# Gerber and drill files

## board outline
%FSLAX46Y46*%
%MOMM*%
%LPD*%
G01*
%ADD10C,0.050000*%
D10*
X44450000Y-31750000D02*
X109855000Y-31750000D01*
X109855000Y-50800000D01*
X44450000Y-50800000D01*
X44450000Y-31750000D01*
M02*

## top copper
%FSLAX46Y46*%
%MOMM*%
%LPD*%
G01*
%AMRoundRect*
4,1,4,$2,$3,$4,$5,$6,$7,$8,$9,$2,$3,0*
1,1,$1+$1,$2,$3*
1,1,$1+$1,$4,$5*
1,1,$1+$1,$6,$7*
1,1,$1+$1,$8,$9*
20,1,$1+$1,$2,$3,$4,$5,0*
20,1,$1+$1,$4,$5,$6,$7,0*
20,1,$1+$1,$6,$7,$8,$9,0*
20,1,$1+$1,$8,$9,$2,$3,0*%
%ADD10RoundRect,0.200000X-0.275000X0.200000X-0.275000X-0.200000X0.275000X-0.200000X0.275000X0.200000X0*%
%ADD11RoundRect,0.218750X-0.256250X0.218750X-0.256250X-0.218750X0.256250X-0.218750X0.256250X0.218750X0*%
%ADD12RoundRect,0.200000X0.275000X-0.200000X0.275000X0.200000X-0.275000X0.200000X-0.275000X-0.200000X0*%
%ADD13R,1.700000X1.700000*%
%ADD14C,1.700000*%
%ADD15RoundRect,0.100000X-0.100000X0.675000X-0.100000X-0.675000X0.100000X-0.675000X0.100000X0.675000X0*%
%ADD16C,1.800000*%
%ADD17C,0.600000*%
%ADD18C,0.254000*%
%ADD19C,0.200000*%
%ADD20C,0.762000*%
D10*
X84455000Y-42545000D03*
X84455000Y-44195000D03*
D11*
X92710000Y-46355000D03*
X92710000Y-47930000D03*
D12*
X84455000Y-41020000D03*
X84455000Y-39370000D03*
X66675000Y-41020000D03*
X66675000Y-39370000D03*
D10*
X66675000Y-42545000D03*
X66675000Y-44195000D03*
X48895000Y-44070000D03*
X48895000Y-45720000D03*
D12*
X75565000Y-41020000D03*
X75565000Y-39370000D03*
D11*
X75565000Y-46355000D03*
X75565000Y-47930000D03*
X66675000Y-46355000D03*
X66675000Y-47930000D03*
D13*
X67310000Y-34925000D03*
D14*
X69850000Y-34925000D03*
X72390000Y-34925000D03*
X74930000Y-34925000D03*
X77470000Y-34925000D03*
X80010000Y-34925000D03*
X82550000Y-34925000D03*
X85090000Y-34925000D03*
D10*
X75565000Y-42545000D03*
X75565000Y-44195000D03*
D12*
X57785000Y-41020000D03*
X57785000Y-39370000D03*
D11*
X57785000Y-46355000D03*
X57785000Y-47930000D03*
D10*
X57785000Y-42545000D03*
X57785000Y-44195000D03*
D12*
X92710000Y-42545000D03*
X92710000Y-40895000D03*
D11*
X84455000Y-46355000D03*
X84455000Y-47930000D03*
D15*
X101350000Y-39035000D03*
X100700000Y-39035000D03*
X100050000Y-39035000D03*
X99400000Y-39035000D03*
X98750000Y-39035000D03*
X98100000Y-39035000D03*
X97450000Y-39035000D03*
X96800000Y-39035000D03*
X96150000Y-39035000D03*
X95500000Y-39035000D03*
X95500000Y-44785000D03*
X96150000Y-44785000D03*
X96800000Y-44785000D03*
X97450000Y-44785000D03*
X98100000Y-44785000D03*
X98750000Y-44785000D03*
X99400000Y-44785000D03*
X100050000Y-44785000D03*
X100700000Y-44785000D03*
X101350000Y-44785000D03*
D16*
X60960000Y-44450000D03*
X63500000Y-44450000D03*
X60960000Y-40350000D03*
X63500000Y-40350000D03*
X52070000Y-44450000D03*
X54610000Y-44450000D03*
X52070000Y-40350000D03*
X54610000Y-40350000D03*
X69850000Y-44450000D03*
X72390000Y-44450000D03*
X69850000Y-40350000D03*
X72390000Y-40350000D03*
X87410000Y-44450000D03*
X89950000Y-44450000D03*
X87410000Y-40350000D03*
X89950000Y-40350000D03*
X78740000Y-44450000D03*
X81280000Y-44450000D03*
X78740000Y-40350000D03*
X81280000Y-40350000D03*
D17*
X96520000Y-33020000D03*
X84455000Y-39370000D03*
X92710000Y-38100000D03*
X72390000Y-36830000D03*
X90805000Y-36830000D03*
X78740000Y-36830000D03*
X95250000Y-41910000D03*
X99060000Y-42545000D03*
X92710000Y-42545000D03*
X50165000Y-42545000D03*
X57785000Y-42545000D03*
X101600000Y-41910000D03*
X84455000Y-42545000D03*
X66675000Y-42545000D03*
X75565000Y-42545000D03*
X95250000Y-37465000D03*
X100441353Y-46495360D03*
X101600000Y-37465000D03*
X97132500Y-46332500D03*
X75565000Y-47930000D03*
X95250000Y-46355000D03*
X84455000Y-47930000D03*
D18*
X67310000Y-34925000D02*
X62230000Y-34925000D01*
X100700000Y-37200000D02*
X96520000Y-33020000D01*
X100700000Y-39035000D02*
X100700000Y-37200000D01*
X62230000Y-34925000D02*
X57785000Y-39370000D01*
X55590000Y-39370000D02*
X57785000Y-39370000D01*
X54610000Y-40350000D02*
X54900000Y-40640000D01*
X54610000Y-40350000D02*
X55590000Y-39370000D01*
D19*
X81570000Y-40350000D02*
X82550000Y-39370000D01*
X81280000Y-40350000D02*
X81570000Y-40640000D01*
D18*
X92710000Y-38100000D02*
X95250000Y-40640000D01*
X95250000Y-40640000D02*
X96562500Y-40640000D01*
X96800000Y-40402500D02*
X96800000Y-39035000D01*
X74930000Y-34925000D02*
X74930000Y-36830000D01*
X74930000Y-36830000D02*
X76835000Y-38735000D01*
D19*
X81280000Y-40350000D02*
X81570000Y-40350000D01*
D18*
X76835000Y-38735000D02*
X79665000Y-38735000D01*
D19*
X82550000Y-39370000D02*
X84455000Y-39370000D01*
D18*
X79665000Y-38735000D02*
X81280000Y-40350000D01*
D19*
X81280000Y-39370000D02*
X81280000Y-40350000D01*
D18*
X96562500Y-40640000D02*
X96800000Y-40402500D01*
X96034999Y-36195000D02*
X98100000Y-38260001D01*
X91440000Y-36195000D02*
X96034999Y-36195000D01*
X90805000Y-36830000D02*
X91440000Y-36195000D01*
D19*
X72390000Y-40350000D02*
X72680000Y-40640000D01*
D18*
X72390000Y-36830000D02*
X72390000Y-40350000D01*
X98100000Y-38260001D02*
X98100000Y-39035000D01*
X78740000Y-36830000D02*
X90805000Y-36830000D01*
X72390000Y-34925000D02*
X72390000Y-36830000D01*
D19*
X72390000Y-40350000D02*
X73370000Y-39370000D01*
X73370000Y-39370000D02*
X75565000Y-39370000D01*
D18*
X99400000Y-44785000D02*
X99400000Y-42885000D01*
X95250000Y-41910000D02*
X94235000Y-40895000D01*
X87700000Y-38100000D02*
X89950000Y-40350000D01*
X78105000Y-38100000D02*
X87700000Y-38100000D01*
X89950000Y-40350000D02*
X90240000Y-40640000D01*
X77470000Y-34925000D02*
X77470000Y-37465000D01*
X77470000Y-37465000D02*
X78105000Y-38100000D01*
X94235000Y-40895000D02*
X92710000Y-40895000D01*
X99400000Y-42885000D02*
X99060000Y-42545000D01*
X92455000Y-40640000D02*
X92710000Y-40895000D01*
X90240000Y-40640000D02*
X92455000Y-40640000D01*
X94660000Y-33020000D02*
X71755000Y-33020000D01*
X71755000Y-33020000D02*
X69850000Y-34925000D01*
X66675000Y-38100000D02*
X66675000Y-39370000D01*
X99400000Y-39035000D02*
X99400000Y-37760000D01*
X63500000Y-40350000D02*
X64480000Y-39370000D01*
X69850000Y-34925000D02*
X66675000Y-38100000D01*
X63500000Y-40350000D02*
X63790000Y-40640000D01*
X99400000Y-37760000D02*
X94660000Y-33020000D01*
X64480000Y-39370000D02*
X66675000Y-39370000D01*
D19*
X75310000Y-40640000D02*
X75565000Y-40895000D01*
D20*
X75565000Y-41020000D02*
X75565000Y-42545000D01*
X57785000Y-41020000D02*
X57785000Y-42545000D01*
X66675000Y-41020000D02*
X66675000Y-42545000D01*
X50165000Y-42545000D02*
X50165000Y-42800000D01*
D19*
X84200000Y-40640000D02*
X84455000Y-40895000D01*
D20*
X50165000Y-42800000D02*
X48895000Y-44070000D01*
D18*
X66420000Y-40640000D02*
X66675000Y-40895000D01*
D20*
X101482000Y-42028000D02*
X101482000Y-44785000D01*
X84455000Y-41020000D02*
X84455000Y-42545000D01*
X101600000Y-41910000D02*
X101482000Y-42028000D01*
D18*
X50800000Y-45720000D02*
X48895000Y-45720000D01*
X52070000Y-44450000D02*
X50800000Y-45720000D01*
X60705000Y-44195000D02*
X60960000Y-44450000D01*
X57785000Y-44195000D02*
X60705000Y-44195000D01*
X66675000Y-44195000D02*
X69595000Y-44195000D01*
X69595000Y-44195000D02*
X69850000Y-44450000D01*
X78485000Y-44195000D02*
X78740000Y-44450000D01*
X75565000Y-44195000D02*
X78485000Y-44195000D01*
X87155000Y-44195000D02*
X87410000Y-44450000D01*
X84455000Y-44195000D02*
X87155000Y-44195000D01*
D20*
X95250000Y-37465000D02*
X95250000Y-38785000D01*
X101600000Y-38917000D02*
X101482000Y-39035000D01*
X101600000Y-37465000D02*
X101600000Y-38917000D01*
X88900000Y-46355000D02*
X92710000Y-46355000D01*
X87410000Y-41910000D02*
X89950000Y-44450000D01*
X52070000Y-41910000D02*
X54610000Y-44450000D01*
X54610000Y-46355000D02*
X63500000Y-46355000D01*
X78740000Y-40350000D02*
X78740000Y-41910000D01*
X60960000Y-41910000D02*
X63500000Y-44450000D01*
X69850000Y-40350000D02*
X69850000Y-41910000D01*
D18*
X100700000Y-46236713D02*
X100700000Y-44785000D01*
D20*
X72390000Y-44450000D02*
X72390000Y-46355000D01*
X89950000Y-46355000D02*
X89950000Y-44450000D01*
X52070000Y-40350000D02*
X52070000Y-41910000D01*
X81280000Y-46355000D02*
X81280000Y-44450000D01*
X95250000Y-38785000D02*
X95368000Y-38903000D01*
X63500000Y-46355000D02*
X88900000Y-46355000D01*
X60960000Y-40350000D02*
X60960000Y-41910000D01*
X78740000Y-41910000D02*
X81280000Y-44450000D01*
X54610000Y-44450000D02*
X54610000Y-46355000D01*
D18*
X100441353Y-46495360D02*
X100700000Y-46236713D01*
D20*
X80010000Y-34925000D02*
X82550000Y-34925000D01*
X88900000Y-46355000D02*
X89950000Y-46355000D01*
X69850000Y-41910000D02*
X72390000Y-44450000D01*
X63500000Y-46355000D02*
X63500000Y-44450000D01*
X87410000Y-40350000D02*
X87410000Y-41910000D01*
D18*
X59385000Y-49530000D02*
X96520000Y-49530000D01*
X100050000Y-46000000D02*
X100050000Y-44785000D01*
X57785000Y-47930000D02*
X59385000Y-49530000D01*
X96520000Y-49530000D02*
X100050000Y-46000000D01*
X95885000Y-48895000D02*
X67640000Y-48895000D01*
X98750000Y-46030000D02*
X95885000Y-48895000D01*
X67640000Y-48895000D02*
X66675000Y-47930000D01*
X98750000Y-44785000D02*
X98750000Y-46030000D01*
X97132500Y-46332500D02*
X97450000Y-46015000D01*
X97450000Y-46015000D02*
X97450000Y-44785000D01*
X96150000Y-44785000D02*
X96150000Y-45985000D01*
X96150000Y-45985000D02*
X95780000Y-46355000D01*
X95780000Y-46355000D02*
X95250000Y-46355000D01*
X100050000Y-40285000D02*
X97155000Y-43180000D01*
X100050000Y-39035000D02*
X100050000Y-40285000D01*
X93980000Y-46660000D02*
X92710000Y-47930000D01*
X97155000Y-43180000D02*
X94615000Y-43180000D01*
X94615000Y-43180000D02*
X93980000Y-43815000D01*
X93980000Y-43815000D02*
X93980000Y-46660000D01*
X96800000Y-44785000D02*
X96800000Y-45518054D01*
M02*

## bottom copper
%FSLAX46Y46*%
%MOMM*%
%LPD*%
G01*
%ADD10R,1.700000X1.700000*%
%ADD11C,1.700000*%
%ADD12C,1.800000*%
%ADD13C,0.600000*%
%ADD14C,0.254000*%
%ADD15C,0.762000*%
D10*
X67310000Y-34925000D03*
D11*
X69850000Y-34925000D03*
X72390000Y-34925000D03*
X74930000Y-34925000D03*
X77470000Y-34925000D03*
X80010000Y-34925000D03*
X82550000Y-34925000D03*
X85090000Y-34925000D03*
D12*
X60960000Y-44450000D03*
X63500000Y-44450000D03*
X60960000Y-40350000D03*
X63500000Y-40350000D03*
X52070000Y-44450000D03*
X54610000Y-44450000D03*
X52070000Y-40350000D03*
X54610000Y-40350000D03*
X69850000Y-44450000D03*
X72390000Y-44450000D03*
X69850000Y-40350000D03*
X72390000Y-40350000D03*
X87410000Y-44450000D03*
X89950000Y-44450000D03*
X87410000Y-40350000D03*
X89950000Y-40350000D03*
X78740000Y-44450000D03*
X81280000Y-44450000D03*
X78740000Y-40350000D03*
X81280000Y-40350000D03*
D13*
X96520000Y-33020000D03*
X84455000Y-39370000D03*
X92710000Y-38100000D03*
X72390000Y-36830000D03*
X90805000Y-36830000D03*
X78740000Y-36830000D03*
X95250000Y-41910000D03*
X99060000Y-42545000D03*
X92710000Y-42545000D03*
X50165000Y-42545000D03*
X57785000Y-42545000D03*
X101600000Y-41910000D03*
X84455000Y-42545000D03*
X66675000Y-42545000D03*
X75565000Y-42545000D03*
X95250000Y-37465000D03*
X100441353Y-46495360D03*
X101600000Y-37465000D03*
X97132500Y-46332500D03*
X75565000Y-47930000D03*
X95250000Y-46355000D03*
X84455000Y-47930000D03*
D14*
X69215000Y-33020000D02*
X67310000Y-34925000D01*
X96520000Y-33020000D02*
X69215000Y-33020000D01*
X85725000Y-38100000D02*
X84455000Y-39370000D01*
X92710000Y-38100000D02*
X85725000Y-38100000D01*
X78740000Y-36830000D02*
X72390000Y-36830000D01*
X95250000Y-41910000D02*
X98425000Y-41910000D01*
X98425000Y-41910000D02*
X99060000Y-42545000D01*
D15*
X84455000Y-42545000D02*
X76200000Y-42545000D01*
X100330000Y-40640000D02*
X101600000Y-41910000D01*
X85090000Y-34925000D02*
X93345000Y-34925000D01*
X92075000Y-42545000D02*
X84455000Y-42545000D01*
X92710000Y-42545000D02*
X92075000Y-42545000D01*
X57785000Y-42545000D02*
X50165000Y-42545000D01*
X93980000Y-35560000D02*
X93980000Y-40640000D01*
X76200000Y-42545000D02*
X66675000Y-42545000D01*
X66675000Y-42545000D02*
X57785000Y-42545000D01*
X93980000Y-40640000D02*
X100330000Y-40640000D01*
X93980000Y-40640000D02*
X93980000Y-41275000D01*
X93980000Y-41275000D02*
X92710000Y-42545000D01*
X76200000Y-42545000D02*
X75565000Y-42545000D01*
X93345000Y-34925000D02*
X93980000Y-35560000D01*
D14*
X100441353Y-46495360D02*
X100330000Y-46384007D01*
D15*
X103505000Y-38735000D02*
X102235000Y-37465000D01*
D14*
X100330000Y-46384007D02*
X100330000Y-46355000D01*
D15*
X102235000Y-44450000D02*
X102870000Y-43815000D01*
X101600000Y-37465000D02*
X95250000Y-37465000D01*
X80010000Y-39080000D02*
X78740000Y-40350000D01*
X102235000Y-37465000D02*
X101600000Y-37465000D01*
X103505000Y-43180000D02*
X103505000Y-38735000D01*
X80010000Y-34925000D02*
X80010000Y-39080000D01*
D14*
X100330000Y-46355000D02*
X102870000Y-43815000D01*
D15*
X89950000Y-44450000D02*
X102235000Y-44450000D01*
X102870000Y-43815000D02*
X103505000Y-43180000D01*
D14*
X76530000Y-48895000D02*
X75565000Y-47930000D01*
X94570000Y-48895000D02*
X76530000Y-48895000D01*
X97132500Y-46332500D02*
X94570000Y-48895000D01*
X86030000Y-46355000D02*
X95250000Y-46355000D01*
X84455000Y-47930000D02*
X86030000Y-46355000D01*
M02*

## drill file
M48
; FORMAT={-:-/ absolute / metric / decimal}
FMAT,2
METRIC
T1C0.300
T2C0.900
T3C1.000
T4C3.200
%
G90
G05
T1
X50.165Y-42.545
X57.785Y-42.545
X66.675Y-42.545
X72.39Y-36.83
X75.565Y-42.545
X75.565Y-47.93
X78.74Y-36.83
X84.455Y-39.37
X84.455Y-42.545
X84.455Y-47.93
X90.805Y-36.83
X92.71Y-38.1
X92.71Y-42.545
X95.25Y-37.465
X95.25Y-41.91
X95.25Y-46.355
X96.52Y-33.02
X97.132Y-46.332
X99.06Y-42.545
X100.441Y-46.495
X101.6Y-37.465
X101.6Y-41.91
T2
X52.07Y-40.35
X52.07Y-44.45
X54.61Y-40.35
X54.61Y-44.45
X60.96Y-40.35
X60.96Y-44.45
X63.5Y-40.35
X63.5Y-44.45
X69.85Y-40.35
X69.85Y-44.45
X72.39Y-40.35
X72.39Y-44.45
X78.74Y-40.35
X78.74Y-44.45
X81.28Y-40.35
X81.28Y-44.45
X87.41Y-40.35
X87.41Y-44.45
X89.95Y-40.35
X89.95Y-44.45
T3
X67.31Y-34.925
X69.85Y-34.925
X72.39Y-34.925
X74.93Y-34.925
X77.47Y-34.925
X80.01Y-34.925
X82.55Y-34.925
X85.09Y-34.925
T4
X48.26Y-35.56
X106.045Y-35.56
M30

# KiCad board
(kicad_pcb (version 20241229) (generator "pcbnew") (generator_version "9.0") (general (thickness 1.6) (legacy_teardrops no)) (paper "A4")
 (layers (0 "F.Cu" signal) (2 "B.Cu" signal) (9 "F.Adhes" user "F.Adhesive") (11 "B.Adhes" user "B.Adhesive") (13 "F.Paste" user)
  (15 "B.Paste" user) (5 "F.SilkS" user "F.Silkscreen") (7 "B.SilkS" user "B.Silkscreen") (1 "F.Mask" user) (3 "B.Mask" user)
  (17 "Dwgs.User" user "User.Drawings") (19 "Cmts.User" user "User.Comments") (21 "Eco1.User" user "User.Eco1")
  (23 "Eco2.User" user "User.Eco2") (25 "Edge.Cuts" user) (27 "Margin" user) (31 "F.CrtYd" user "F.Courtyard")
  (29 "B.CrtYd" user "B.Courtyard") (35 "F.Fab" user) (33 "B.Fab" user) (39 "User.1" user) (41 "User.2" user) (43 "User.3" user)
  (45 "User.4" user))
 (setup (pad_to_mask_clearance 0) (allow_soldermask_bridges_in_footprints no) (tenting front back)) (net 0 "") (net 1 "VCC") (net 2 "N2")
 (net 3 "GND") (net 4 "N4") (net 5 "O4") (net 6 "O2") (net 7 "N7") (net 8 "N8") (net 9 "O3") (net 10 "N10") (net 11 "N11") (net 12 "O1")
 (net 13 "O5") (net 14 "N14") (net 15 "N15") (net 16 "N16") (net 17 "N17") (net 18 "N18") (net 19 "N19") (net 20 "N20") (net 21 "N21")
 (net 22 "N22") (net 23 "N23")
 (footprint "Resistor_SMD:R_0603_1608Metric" (layer "F.Cu") (at 84.455 43.37 -90)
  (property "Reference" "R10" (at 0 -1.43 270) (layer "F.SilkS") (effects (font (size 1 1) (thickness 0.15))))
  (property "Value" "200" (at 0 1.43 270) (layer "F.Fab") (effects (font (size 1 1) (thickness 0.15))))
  (pad "1" smd roundrect (at -0.825 0 270) (size 0.8 0.95) (layers "F.Cu" "F.Mask" "F.Paste") (roundrect_rratio 0.25) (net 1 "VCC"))
  (pad "2" smd roundrect (at 0.825 0 270) (size 0.8 0.95) (layers "F.Cu" "F.Mask" "F.Paste") (roundrect_rratio 0.25) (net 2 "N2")))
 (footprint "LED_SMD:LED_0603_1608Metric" (layer "F.Cu") (at 92.71 47.1425 -90)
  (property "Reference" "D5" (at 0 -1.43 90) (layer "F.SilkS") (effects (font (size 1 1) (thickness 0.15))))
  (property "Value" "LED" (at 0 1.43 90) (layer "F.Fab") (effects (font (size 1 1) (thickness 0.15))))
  (pad "1" smd roundrect (at -0.7875 0 270) (size 0.875 0.95) (layers "F.Cu" "F.Mask" "F.Paste") (roundrect_rratio 0.25) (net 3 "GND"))
  (pad "2" smd roundrect (at 0.7875 0 270) (size 0.875 0.95) (layers "F.Cu" "F.Mask" "F.Paste") (roundrect_rratio 0.25) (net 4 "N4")))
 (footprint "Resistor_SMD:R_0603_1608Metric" (layer "F.Cu") (at 84.455 40.195 90)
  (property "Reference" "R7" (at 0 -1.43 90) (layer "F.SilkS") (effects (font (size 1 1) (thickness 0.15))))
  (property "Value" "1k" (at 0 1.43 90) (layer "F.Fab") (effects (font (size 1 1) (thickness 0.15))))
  (pad "1" smd roundrect (at -0.825 0 90) (size 0.8 0.95) (layers "F.Cu" "F.Mask" "F.Paste") (roundrect_rratio 0.25) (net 1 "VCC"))
  (pad "2" smd roundrect (at 0.825 0 90) (size 0.8 0.95) (layers "F.Cu" "F.Mask" "F.Paste") (roundrect_rratio 0.25) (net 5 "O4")))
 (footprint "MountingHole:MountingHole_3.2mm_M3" (layer "F.Cu") (at 106.045 35.56)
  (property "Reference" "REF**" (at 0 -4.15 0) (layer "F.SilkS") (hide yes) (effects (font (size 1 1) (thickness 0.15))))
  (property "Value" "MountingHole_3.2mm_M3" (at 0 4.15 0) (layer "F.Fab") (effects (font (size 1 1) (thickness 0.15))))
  (pad "" np_thru_hole circle (at 0 0) (size 3.2 3.2) (drill 3.2) (layers "*.Cu" "*.Mask")))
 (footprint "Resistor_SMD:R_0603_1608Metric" (layer "F.Cu") (at 66.675 40.195 90)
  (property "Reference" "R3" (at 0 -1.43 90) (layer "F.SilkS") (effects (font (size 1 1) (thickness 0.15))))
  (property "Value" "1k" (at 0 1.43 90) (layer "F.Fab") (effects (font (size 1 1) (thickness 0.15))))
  (pad "1" smd roundrect (at -0.825 0 90) (size 0.8 0.95) (layers "F.Cu" "F.Mask" "F.Paste") (roundrect_rratio 0.25) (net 1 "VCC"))
  (pad "2" smd roundrect (at 0.825 0 90) (size 0.8 0.95) (layers "F.Cu" "F.Mask" "F.Paste") (roundrect_rratio 0.25) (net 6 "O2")))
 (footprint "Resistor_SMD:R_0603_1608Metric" (layer "F.Cu") (at 66.675 43.37 -90)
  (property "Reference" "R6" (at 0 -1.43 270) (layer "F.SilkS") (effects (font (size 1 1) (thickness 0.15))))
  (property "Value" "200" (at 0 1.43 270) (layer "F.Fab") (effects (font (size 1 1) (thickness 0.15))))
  (pad "1" smd roundrect (at -0.825 0 270) (size 0.8 0.95) (layers "F.Cu" "F.Mask" "F.Paste") (roundrect_rratio 0.25) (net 1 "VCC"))
  (pad "2" smd roundrect (at 0.825 0 270) (size 0.8 0.95) (layers "F.Cu" "F.Mask" "F.Paste") (roundrect_rratio 0.25) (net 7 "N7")))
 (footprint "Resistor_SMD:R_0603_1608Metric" (layer "F.Cu") (at 48.895 44.895 -90)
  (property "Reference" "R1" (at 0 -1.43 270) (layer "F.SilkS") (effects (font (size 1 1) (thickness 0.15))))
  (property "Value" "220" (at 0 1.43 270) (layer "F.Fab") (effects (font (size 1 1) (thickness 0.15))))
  (pad "1" smd roundrect (at -0.825 0 270) (size 0.8 0.95) (layers "F.Cu" "F.Mask" "F.Paste") (roundrect_rratio 0.25) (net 1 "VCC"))
  (pad "2" smd roundrect (at 0.825 0 270) (size 0.8 0.95) (layers "F.Cu" "F.Mask" "F.Paste") (roundrect_rratio 0.25) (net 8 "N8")))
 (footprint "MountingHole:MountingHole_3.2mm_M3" (layer "F.Cu") (at 48.26 35.56)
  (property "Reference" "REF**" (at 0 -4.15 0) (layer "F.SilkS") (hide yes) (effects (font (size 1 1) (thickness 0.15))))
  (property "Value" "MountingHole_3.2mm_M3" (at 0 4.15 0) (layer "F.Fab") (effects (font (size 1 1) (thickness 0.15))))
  (pad "" np_thru_hole circle (at 0 0) (size 3.2 3.2) (drill 3.2) (layers "*.Cu" "*.Mask")))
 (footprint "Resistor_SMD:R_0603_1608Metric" (layer "F.Cu") (at 75.565 40.195 90)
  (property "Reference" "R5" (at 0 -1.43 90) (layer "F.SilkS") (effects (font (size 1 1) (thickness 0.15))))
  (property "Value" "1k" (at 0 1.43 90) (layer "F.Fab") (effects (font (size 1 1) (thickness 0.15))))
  (pad "1" smd roundrect (at -0.825 0 90) (size 0.8 0.95) (layers "F.Cu" "F.Mask" "F.Paste") (roundrect_rratio 0.25) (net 1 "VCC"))
  (pad "2" smd roundrect (at 0.825 0 90) (size 0.8 0.95) (layers "F.Cu" "F.Mask" "F.Paste") (roundrect_rratio 0.25) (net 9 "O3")))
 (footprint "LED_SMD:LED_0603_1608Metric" (layer "F.Cu") (at 75.565 47.1425 -90)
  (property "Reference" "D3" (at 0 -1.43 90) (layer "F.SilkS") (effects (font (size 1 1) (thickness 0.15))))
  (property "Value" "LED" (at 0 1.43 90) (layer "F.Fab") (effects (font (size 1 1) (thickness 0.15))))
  (pad "1" smd roundrect (at -0.7875 0 270) (size 0.875 0.95) (layers "F.Cu" "F.Mask" "F.Paste") (roundrect_rratio 0.25) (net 3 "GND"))
  (pad "2" smd roundrect (at 0.7875 0 270) (size 0.875 0.95) (layers "F.Cu" "F.Mask" "F.Paste") (roundrect_rratio 0.25) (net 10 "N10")))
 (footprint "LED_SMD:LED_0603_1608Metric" (layer "F.Cu") (at 66.675 47.1425 -90)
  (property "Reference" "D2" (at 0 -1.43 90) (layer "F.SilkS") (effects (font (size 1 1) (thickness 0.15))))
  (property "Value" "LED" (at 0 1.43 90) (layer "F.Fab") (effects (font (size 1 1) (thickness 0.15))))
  (pad "1" smd roundrect (at -0.7875 0 270) (size 0.875 0.95) (layers "F.Cu" "F.Mask" "F.Paste") (roundrect_rratio 0.25) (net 3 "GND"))
  (pad "2" smd roundrect (at 0.7875 0 270) (size 0.875 0.95) (layers "F.Cu" "F.Mask" "F.Paste") (roundrect_rratio 0.25) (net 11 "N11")))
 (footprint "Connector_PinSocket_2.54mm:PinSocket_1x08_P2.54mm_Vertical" (layer "F.Cu") (at 67.31 34.925 90)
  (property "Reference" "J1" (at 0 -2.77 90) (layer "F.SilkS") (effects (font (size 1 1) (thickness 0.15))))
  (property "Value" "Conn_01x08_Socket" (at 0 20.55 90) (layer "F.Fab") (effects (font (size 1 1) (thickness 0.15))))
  (pad "1" thru_hole rect (at 0 0 90) (size 1.7 1.7) (drill 1) (layers "*.Cu" "*.Mask") (remove_unused_layers no) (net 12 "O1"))
  (pad "2" thru_hole circle (at 0 2.54 90) (size 1.7 1.7) (drill 1) (layers "*.Cu" "*.Mask") (remove_unused_layers no) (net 6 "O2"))
  (pad "3" thru_hole circle (at 0 5.08 90) (size 1.7 1.7) (drill 1) (layers "*.Cu" "*.Mask") (remove_unused_layers no) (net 9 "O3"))
  (pad "4" thru_hole circle (at 0 7.62 90) (size 1.7 1.7) (drill 1) (layers "*.Cu" "*.Mask") (remove_unused_layers no) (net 5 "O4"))
  (pad "5" thru_hole circle (at 0 10.16 90) (size 1.7 1.7) (drill 1) (layers "*.Cu" "*.Mask") (remove_unused_layers no) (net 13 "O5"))
  (pad "6" thru_hole circle (at 0 12.7 90) (size 1.7 1.7) (drill 1) (layers "*.Cu" "*.Mask") (remove_unused_layers no) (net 3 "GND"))
  (pad "7" thru_hole circle (at 0 15.24 90) (size 1.7 1.7) (drill 1) (layers "*.Cu" "*.Mask") (remove_unused_layers no) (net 3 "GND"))
  (pad "8" thru_hole circle (at 0 17.78 90) (size 1.7 1.7) (drill 1) (layers "*.Cu" "*.Mask") (remove_unused_layers no) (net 1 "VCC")))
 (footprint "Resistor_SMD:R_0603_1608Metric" (layer "F.Cu") (at 75.565 43.37 -90)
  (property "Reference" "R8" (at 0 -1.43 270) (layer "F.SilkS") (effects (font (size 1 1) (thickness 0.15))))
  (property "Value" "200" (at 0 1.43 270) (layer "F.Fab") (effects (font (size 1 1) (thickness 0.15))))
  (pad "1" smd roundrect (at -0.825 0 270) (size 0.8 0.95) (layers "F.Cu" "F.Mask" "F.Paste") (roundrect_rratio 0.25) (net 1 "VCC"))
  (pad "2" smd roundrect (at 0.825 0 270) (size 0.8 0.95) (layers "F.Cu" "F.Mask" "F.Paste") (roundrect_rratio 0.25) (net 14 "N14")))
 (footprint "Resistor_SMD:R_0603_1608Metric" (layer "F.Cu") (at 57.785 40.195 90)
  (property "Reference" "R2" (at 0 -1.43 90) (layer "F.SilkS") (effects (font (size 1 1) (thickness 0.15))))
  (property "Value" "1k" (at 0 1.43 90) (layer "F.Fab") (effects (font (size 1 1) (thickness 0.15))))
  (pad "1" smd roundrect (at -0.825 0 90) (size 0.8 0.95) (layers "F.Cu" "F.Mask" "F.Paste") (roundrect_rratio 0.25) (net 1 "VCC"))
  (pad "2" smd roundrect (at 0.825 0 90) (size 0.8 0.95) (layers "F.Cu" "F.Mask" "F.Paste") (roundrect_rratio 0.25) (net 12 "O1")))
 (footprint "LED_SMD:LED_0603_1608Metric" (layer "F.Cu") (at 57.785 47.1425 -90)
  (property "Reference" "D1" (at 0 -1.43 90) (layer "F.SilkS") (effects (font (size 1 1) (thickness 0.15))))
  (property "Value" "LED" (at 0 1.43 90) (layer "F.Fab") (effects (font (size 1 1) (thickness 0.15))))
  (pad "1" smd roundrect (at -0.7875 0 270) (size 0.875 0.95) (layers "F.Cu" "F.Mask" "F.Paste") (roundrect_rratio 0.25) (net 3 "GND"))
  (pad "2" smd roundrect (at 0.7875 0 270) (size 0.875 0.95) (layers "F.Cu" "F.Mask" "F.Paste") (roundrect_rratio 0.25) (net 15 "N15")))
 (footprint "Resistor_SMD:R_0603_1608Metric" (layer "F.Cu") (at 57.785 43.37 -90)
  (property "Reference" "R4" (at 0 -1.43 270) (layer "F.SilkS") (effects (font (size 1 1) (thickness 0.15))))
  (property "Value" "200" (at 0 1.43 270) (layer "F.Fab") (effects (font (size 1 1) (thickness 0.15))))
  (pad "1" smd roundrect (at -0.825 0 270) (size 0.8 0.95) (layers "F.Cu" "F.Mask" "F.Paste") (roundrect_rratio 0.25) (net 1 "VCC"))
  (pad "2" smd roundrect (at 0.825 0 270) (size 0.8 0.95) (layers "F.Cu" "F.Mask" "F.Paste") (roundrect_rratio 0.25) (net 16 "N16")))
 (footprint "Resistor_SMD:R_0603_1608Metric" (layer "F.Cu") (at 92.71 41.72 90)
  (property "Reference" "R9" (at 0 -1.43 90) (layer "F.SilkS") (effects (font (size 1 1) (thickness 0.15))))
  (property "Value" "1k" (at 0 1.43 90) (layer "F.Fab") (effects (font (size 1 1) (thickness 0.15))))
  (pad "1" smd roundrect (at -0.825 0 90) (size 0.8 0.95) (layers "F.Cu" "F.Mask" "F.Paste") (roundrect_rratio 0.25) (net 1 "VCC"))
  (pad "2" smd roundrect (at 0.825 0 90) (size 0.8 0.95) (layers "F.Cu" "F.Mask" "F.Paste") (roundrect_rratio 0.25) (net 13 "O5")))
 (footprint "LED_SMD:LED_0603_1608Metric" (layer "F.Cu") (at 84.455 47.1425 -90)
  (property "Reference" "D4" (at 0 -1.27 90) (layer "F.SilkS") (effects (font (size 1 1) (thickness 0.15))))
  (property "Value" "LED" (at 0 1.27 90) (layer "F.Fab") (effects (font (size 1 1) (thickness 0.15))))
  (pad "1" smd roundrect (at -0.7875 0 270) (size 0.875 0.95) (layers "F.Cu" "F.Mask" "F.Paste") (roundrect_rratio 0.25) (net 3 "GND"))
  (pad "2" smd roundrect (at 0.7875 0 270) (size 0.875 0.95) (layers "F.Cu" "F.Mask" "F.Paste") (roundrect_rratio 0.25) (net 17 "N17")))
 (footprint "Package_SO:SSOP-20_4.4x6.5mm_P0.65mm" (layer "F.Cu") (at 98.425 41.91 -90)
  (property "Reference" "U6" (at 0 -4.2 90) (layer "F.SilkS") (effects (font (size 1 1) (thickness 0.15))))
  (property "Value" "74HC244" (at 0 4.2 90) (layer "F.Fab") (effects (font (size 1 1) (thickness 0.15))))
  (pad "1" smd roundrect (at -2.875 -2.925 270) (size 1.55 0.4) (layers "F.Cu" "F.Mask" "F.Paste") (roundrect_rratio 0.25) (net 3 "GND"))
  (pad "2" smd roundrect (at -2.875 -2.275 270) (size 1.55 0.4) (layers "F.Cu" "F.Mask" "F.Paste") (roundrect_rratio 0.25) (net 12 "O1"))
  (pad "3" smd roundrect (at -2.875 -1.625 270) (size 1.55 0.4) (layers "F.Cu" "F.Mask" "F.Paste") (roundrect_rratio 0.25) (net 4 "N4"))
  (pad "4" smd roundrect (at -2.875 -0.975 270) (size 1.55 0.4) (layers "F.Cu" "F.Mask" "F.Paste") (roundrect_rratio 0.25) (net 6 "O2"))
  (pad "5" smd roundrect (at -2.875 -0.325 270) (size 1.55 0.4) (layers "F.Cu" "F.Mask" "F.Paste") (roundrect_rratio 0.25) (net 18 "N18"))
  (pad "6" smd roundrect (at -2.875 0.325 270) (size 1.55 0.4) (layers "F.Cu" "F.Mask" "F.Paste") (roundrect_rratio 0.25) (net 9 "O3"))
  (pad "7" smd roundrect (at -2.875 0.975 270) (size 1.55 0.4) (layers "F.Cu" "F.Mask" "F.Paste") (roundrect_rratio 0.25) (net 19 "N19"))
  (pad "8" smd roundrect (at -2.875 1.625 270) (size 1.55 0.4) (layers "F.Cu" "F.Mask" "F.Paste") (roundrect_rratio 0.25) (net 5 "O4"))
  (pad "9" smd roundrect (at -2.875 2.275 270) (size 1.55 0.4) (layers "F.Cu" "F.Mask" "F.Paste") (roundrect_rratio 0.25) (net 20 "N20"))
  (pad "10" smd roundrect (at -2.875 2.925 270) (size 1.55 0.4) (layers "F.Cu" "F.Mask" "F.Paste") (roundrect_rratio 0.25) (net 3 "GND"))
  (pad "11" smd roundrect (at 2.875 2.925 270) (size 1.55 0.4) (layers "F.Cu" "F.Mask" "F.Paste") (roundrect_rratio 0.25) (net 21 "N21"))
  (pad "12" smd roundrect (at 2.875 2.275 270) (size 1.55 0.4) (layers "F.Cu" "F.Mask" "F.Paste") (roundrect_rratio 0.25) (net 17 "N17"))
  (pad "13" smd roundrect (at 2.875 1.625 270) (size 1.55 0.4) (layers "F.Cu" "F.Mask" "F.Paste") (roundrect_rratio 0.25) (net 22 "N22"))
  (pad "14" smd roundrect (at 2.875 0.975 270) (size 1.55 0.4) (layers "F.Cu" "F.Mask" "F.Paste") (roundrect_rratio 0.25) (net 10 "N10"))
  (pad "15" smd roundrect (at 2.875 0.325 270) (size 1.55 0.4) (layers "F.Cu" "F.Mask" "F.Paste") (roundrect_rratio 0.25) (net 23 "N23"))
  (pad "16" smd roundrect (at 2.875 -0.325 270) (size 1.55 0.4) (layers "F.Cu" "F.Mask" "F.Paste") (roundrect_rratio 0.25) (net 11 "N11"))
  (pad "17" smd roundrect (at 2.875 -0.975 270) (size 1.55 0.4) (layers "F.Cu" "F.Mask" "F.Paste") (roundrect_rratio 0.25) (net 13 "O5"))
  (pad "18" smd roundrect (at 2.875 -1.625 270) (size 1.55 0.4) (layers "F.Cu" "F.Mask" "F.Paste") (roundrect_rratio 0.25) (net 15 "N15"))
  (pad "19" smd roundrect (at 2.875 -2.275 270) (size 1.55 0.4) (layers "F.Cu" "F.Mask" "F.Paste") (roundrect_rratio 0.25) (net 3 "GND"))
  (pad "20" smd roundrect (at 2.875 -2.925 270) (size 1.55 0.4) (layers "F.Cu" "F.Mask" "F.Paste") (roundrect_rratio 0.25) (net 1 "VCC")))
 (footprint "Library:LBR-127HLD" (layer "B.Cu") (at 62.23 42.4 -90)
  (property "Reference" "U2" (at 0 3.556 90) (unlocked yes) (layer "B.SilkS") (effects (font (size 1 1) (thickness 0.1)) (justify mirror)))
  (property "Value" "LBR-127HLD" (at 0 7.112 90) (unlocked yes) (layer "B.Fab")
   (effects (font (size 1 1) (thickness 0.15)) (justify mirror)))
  (pad "1" thru_hole circle (at 2.05 1.27 270) (size 1.8 1.8) (drill 0.9) (layers "*.Cu" "*.Mask") (remove_unused_layers no) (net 16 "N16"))
  (pad "2" thru_hole circle (at 2.05 -1.27 270) (size 1.8 1.8) (drill 0.9) (layers "*.Cu" "*.Mask") (remove_unused_layers no) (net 3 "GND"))
  (pad "3" thru_hole circle (at -2.05 1.27 270) (size 1.8 1.8) (drill 0.9) (layers "*.Cu" "*.Mask") (remove_unused_layers no) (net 3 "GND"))
  (pad "4" thru_hole circle (at -2.05 -1.27 270) (size 1.8 1.8) (drill 0.9) (layers "*.Cu" "*.Mask") (remove_unused_layers no) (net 6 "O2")))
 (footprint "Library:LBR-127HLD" (layer "B.Cu") (at 53.34 42.4 -90)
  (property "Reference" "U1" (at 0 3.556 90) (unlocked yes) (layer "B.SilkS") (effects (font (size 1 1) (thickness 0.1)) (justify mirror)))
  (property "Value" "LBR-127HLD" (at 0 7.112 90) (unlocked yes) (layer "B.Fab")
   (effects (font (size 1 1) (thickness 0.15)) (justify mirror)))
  (pad "1" thru_hole circle (at 2.05 1.27 270) (size 1.8 1.8) (drill 0.9) (layers "*.Cu" "*.Mask") (remove_unused_layers no) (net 8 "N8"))
  (pad "2" thru_hole circle (at 2.05 -1.27 270) (size 1.8 1.8) (drill 0.9) (layers "*.Cu" "*.Mask") (remove_unused_layers no) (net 3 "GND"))
  (pad "3" thru_hole circle (at -2.05 1.27 270) (size 1.8 1.8) (drill 0.9) (layers "*.Cu" "*.Mask") (remove_unused_layers no) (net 3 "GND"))
  (pad "4" thru_hole circle (at -2.05 -1.27 270) (size 1.8 1.8) (drill 0.9) (layers "*.Cu" "*.Mask") (remove_unused_layers no) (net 12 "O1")))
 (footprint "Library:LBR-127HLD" (layer "B.Cu") (at 71.12 42.4 -90)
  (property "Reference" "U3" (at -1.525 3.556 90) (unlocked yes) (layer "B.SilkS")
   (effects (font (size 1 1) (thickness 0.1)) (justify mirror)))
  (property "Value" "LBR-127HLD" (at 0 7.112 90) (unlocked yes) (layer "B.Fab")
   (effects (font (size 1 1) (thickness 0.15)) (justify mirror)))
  (pad "1" thru_hole circle (at 2.05 1.27 270) (size 1.8 1.8) (drill 0.9) (layers "*.Cu" "*.Mask") (remove_unused_layers no) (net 7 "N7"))
  (pad "2" thru_hole circle (at 2.05 -1.27 270) (size 1.8 1.8) (drill 0.9) (layers "*.Cu" "*.Mask") (remove_unused_layers no) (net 3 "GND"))
  (pad "3" thru_hole circle (at -2.05 1.27 270) (size 1.8 1.8) (drill 0.9) (layers "*.Cu" "*.Mask") (remove_unused_layers no) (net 3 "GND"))
  (pad "4" thru_hole circle (at -2.05 -1.27 270) (size 1.8 1.8) (drill 0.9) (layers "*.Cu" "*.Mask") (remove_unused_layers no) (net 9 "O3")))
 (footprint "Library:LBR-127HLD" (layer "B.Cu") (at 88.68 42.4 -90)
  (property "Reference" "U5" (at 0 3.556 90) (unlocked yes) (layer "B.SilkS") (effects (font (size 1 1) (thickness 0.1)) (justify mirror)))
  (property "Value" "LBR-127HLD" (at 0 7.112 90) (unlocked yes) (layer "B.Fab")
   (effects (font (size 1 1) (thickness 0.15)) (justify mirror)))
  (pad "1" thru_hole circle (at 2.05 1.27 270) (size 1.8 1.8) (drill 0.9) (layers "*.Cu" "*.Mask") (remove_unused_layers no) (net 2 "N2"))
  (pad "2" thru_hole circle (at 2.05 -1.27 270) (size 1.8 1.8) (drill 0.9) (layers "*.Cu" "*.Mask") (remove_unused_layers no) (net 3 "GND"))
  (pad "3" thru_hole circle (at -2.05 1.27 270) (size 1.8 1.8) (drill 0.9) (layers "*.Cu" "*.Mask") (remove_unused_layers no) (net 3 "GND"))
  (pad "4" thru_hole circle (at -2.05 -1.27 270) (size 1.8 1.8) (drill 0.9) (layers "*.Cu" "*.Mask") (remove_unused_layers no) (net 13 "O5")))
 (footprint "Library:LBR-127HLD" (layer "B.Cu") (at 80.01 42.4 -90)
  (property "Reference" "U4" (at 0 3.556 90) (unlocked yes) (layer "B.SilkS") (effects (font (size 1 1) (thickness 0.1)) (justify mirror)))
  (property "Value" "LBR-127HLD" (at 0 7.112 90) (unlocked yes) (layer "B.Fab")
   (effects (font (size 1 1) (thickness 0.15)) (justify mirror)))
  (pad "1" thru_hole circle (at 2.05 1.27 270) (size 1.8 1.8) (drill 0.9) (layers "*.Cu" "*.Mask") (remove_unused_layers no) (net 14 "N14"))
  (pad "2" thru_hole circle (at 2.05 -1.27 270) (size 1.8 1.8) (drill 0.9) (layers "*.Cu" "*.Mask") (remove_unused_layers no) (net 3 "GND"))
  (pad "3" thru_hole circle (at -2.05 1.27 270) (size 1.8 1.8) (drill 0.9) (layers "*.Cu" "*.Mask") (remove_unused_layers no) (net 3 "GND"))
  (pad "4" thru_hole circle (at -2.05 -1.27 270) (size 1.8 1.8) (drill 0.9) (layers "*.Cu" "*.Mask") (remove_unused_layers no) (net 5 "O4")))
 (gr_rect (start 44.45 31.75) (end 109.855 50.8) (stroke (width 0.05) (type default)) (fill no) (layer "Edge.Cuts"))
 (segment (start 67.31 34.925) (end 62.23 34.925) (width 0.254) (layer "F.Cu") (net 12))
 (segment (start 100.7 37.2) (end 96.52 33.02) (width 0.254) (layer "F.Cu") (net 12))
 (segment (start 100.7 39.035) (end 100.7 37.2) (width 0.254) (layer "F.Cu") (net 12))
 (segment (start 62.23 34.925) (end 57.785 39.37) (width 0.254) (layer "F.Cu") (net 12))
 (segment (start 55.59 39.37) (end 57.785 39.37) (width 0.254) (layer "F.Cu") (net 12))
 (segment (start 54.61 40.35) (end 54.9 40.64) (width 0.254) (layer "F.Cu") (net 12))
 (segment (start 54.61 40.35) (end 55.59 39.37) (width 0.254) (layer "F.Cu") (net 12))
 (via (at 96.52 33.02) (size 0.6) (drill 0.3) (layers "F.Cu" "B.Cu") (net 12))
 (segment (start 69.215 33.02) (end 67.31 34.925) (width 0.254) (layer "B.Cu") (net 12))
 (segment (start 96.52 33.02) (end 69.215 33.02) (width 0.254) (layer "B.Cu") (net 12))
 (segment (start 81.57 40.35) (end 82.55 39.37) (width 0.2) (layer "F.Cu") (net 5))
 (segment (start 81.28 40.35) (end 81.57 40.64) (width 0.2) (layer "F.Cu") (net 5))
 (segment (start 92.71 38.1) (end 95.25 40.64) (width 0.254) (layer "F.Cu") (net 5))
 (segment (start 95.25 40.64) (end 96.5625 40.64) (width 0.254) (layer "F.Cu") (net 5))
 (segment (start 96.8 40.4025) (end 96.8 39.035) (width 0.254) (layer "F.Cu") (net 5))
 (segment (start 74.93 34.925) (end 74.93 36.83) (width 0.254) (layer "F.Cu") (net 5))
 (segment (start 74.93 36.83) (end 76.835 38.735) (width 0.254) (layer "F.Cu") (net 5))
 (segment (start 81.28 40.35) (end 81.57 40.35) (width 0.2) (layer "F.Cu") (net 5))
 (segment (start 76.835 38.735) (end 79.665 38.735) (width 0.254) (layer "F.Cu") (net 5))
 (segment (start 82.55 39.37) (end 84.455 39.37) (width 0.2) (layer "F.Cu") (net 5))
 (segment (start 79.665 38.735) (end 81.28 40.35) (width 0.254) (layer "F.Cu") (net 5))
 (segment (start 81.28 39.37) (end 81.28 40.35) (width 0.2) (layer "F.Cu") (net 5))
 (segment (start 96.5625 40.64) (end 96.8 40.4025) (width 0.254) (layer "F.Cu") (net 5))
 (via (at 84.455 39.37) (size 0.6) (drill 0.3) (layers "F.Cu" "B.Cu") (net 5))
 (via (at 92.71 38.1) (size 0.6) (drill 0.3) (layers "F.Cu" "B.Cu") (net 5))
 (segment (start 85.725 38.1) (end 84.455 39.37) (width 0.254) (layer "B.Cu") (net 5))
 (segment (start 92.71 38.1) (end 85.725 38.1) (width 0.254) (layer "B.Cu") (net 5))
 (segment (start 96.034999 36.195) (end 98.1 38.260001) (width 0.254) (layer "F.Cu") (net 9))
 (segment (start 91.44 36.195) (end 96.034999 36.195) (width 0.254) (layer "F.Cu") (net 9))
 (segment (start 90.805 36.83) (end 91.44 36.195) (width 0.254) (layer "F.Cu") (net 9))
 (segment (start 72.39 40.35) (end 72.68 40.64) (width 0.2) (layer "F.Cu") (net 9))
 (segment (start 72.39 36.83) (end 72.39 40.35) (width 0.254) (layer "F.Cu") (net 9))
 (segment (start 98.1 38.260001) (end 98.1 39.035) (width 0.254) (layer "F.Cu") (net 9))
 (segment (start 78.74 36.83) (end 90.805 36.83) (width 0.254) (layer "F.Cu") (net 9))
 (segment (start 72.39 34.925) (end 72.39 36.83) (width 0.254) (layer "F.Cu") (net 9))
 (segment (start 72.39 40.35) (end 73.37 39.37) (width 0.2) (layer "F.Cu") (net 9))
 (segment (start 73.37 39.37) (end 75.565 39.37) (width 0.2) (layer "F.Cu") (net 9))
 (via (at 72.39 36.83) (size 0.6) (drill 0.3) (layers "F.Cu" "B.Cu") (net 9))
 (via (at 90.805 36.83) (size 0.6) (drill 0.3) (layers "F.Cu" "B.Cu") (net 9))
 (via (at 78.74 36.83) (size 0.6) (drill 0.3) (layers "F.Cu" "B.Cu") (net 9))
 (segment (start 78.74 36.83) (end 72.39 36.83) (width 0.254) (layer "B.Cu") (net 9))
 (segment (start 99.4 44.785) (end 99.4 42.885) (width 0.254) (layer "F.Cu") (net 13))
 (segment (start 95.25 41.91) (end 94.235 40.895) (width 0.254) (layer "F.Cu") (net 13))
 (segment (start 87.7 38.1) (end 89.95 40.35) (width 0.254) (layer "F.Cu") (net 13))
 (segment (start 78.105 38.1) (end 87.7 38.1) (width 0.254) (layer "F.Cu") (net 13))
 (segment (start 89.95 40.35) (end 90.24 40.64) (width 0.254) (layer "F.Cu") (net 13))
 (segment (start 77.47 34.925) (end 77.47 37.465) (width 0.254) (layer "F.Cu") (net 13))
 (segment (start 77.47 37.465) (end 78.105 38.1) (width 0.254) (layer "F.Cu") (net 13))
 (segment (start 94.235 40.895) (end 92.71 40.895) (width 0.254) (layer "F.Cu") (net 13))
 (segment (start 99.4 42.885) (end 99.06 42.545) (width 0.254) (layer "F.Cu") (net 13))
 (segment (start 92.455 40.64) (end 92.71 40.895) (width 0.254) (layer "F.Cu") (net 13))
 (segment (start 90.24 40.64) (end 92.455 40.64) (width 0.254) (layer "F.Cu") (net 13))
 (via (at 95.25 41.91) (size 0.6) (drill 0.3) (layers "F.Cu" "B.Cu") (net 13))
 (via (at 99.06 42.545) (size 0.6) (drill 0.3) (layers "F.Cu" "B.Cu") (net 13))
 (segment (start 95.25 41.91) (end 98.425 41.91) (width 0.254) (layer "B.Cu") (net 13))
 (segment (start 98.425 41.91) (end 99.06 42.545) (width 0.254) (layer "B.Cu") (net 13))
 (segment (start 94.66 33.02) (end 71.755 33.02) (width 0.254) (layer "F.Cu") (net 6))
 (segment (start 71.755 33.02) (end 69.85 34.925) (width 0.254) (layer "F.Cu") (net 6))
 (segment (start 66.675 38.1) (end 66.675 39.37) (width 0.254) (layer "F.Cu") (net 6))
 (segment (start 99.4 39.035) (end 99.4 37.76) (width 0.254) (layer "F.Cu") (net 6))
 (segment (start 63.5 40.35) (end 64.48 39.37) (width 0.254) (layer "F.Cu") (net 6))
 (segment (start 69.85 34.925) (end 66.675 38.1) (width 0.254) (layer "F.Cu") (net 6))
 (segment (start 63.5 40.35) (end 63.79 40.64) (width 0.254) (layer "F.Cu") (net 6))
 (segment (start 99.4 37.76) (end 94.66 33.02) (width 0.254) (layer "F.Cu") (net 6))
 (segment (start 64.48 39.37) (end 66.675 39.37) (width 0.254) (layer "F.Cu") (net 6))
 (segment (start 75.31 40.64) (end 75.565 40.895) (width 0.2) (layer "F.Cu") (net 1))
 (segment (start 75.565 41.02) (end 75.565 42.545) (width 0.762) (layer "F.Cu") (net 1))
 (segment (start 57.785 41.02) (end 57.785 42.545) (width 0.762) (layer "F.Cu") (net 1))
 (segment (start 66.675 41.02) (end 66.675 42.545) (width 0.762) (layer "F.Cu") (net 1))
 (segment (start 50.165 42.545) (end 50.165 42.8) (width 0.762) (layer "F.Cu") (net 1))
 (segment (start 84.2 40.64) (end 84.455 40.895) (width 0.2) (layer "F.Cu") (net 1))
 (segment (start 50.165 42.8) (end 48.895 44.07) (width 0.762) (layer "F.Cu") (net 1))
 (segment (start 66.42 40.64) (end 66.675 40.895) (width 0.254) (layer "F.Cu") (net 1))
 (segment (start 101.482 42.028) (end 101.482 44.785) (width 0.762) (layer "F.Cu") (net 1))
 (segment (start 84.455 41.02) (end 84.455 42.545) (width 0.762) (layer "F.Cu") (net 1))
 (segment (start 101.6 41.91) (end 101.482 42.028) (width 0.762) (layer "F.Cu") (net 1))
 (via (at 92.71 42.545) (size 0.6) (drill 0.3) (layers "F.Cu" "B.Cu") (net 1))
 (via (at 50.165 42.545) (size 0.6) (drill 0.3) (layers "F.Cu" "B.Cu") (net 1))
 (via (at 57.785 42.545) (size 0.6) (drill 0.3) (layers "F.Cu" "B.Cu") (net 1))
 (via (at 101.6 41.91) (size 0.6) (drill 0.3) (layers "F.Cu" "B.Cu") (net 1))
 (via (at 84.455 42.545) (size 0.6) (drill 0.3) (layers "F.Cu" "B.Cu") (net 1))
 (via (at 66.675 42.545) (size 0.6) (drill 0.3) (layers "F.Cu" "B.Cu") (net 1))
 (via (at 75.565 42.545) (size 0.6) (drill 0.3) (layers "F.Cu" "B.Cu") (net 1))
 (segment (start 84.455 42.545) (end 76.2 42.545) (width 0.762) (layer "B.Cu") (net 1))
 (segment (start 100.33 40.64) (end 101.6 41.91) (width 0.762) (layer "B.Cu") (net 1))
 (segment (start 85.09 34.925) (end 93.345 34.925) (width 0.762) (layer "B.Cu") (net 1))
 (segment (start 92.075 42.545) (end 84.455 42.545) (width 0.762) (layer "B.Cu") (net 1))
 (segment (start 92.71 42.545) (end 92.075 42.545) (width 0.762) (layer "B.Cu") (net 1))
 (segment (start 57.785 42.545) (end 50.165 42.545) (width 0.762) (layer "B.Cu") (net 1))
 (segment (start 93.98 35.56) (end 93.98 40.64) (width 0.762) (layer "B.Cu") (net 1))
 (segment (start 76.2 42.545) (end 66.675 42.545) (width 0.762) (layer "B.Cu") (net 1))
 (segment (start 66.675 42.545) (end 57.785 42.545) (width 0.762) (layer "B.Cu") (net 1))
 (segment (start 93.98 40.64) (end 100.33 40.64) (width 0.762) (layer "B.Cu") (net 1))
 (segment (start 93.98 40.64) (end 93.98 41.275) (width 0.762) (layer "B.Cu") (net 1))
 (segment (start 93.98 41.275) (end 92.71 42.545) (width 0.762) (layer "B.Cu") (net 1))
 (segment (start 76.2 42.545) (end 75.565 42.545) (width 0.762) (layer "B.Cu") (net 1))
 (segment (start 93.345 34.925) (end 93.98 35.56) (width 0.762) (layer "B.Cu") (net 1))
 (segment (start 50.8 45.72) (end 48.895 45.72) (width 0.254) (layer "F.Cu") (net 8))
 (segment (start 52.07 44.45) (end 50.8 45.72) (width 0.254) (layer "F.Cu") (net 8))
 (segment (start 60.705 44.195) (end 60.96 44.45) (width 0.254) (layer "F.Cu") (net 16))
 (segment (start 57.785 44.195) (end 60.705 44.195) (width 0.254) (layer "F.Cu") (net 16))
 (segment (start 66.675 44.195) (end 69.595 44.195) (width 0.254) (layer "F.Cu") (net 7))
 (segment (start 69.595 44.195) (end 69.85 44.45) (width 0.254) (layer "F.Cu") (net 7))
 (segment (start 78.485 44.195) (end 78.74 44.45) (width 0.254) (layer "F.Cu") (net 14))
 (segment (start 75.565 44.195) (end 78.485 44.195) (width 0.254) (layer "F.Cu") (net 14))
 (segment (start 87.155 44.195) (end 87.41 44.45) (width 0.254) (layer "F.Cu") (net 2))
 (segment (start 84.455 44.195) (end 87.155 44.195) (width 0.254) (layer "F.Cu") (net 2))
 (segment (start 95.25 37.465) (end 95.25 38.785) (width 0.762) (layer "F.Cu") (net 3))
 (segment (start 101.6 38.917) (end 101.482 39.035) (width 0.762) (layer "F.Cu") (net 3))
 (segment (start 101.6 37.465) (end 101.6 38.917) (width 0.762) (layer "F.Cu") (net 3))
 (segment (start 88.9 46.355) (end 92.71 46.355) (width 0.762) (layer "F.Cu") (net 3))
 (segment (start 87.41 41.91) (end 89.95 44.45) (width 0.762) (layer "F.Cu") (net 3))
 (segment (start 52.07 41.91) (end 54.61 44.45) (width 0.762) (layer "F.Cu") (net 3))
 (segment (start 54.61 46.355) (end 63.5 46.355) (width 0.762) (layer "F.Cu") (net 3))
 (segment (start 78.74 40.35) (end 78.74 41.91) (width 0.762) (layer "F.Cu") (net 3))
 (segment (start 60.96 41.91) (end 63.5 44.45) (width 0.762) (layer "F.Cu") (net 3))
 (segment (start 69.85 40.35) (end 69.85 41.91) (width 0.762) (layer "F.Cu") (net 3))
 (segment (start 100.7 46.236713) (end 100.7 44.785) (width 0.254) (layer "F.Cu") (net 3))
 (segment (start 72.39 44.45) (end 72.39 46.355) (width 0.762) (layer "F.Cu") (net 3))
 (segment (start 89.95 46.355) (end 89.95 44.45) (width 0.762) (layer "F.Cu") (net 3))
 (segment (start 52.07 40.35) (end 52.07 41.91) (width 0.762) (layer "F.Cu") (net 3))
 (segment (start 81.28 46.355) (end 81.28 44.45) (width 0.762) (layer "F.Cu") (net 3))
 (segment (start 95.25 38.785) (end 95.368 38.903) (width 0.762) (layer "F.Cu") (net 3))
 (segment (start 63.5 46.355) (end 88.9 46.355) (width 0.762) (layer "F.Cu") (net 3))
 (segment (start 60.96 40.35) (end 60.96 41.91) (width 0.762) (layer "F.Cu") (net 3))
 (segment (start 78.74 41.91) (end 81.28 44.45) (width 0.762) (layer "F.Cu") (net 3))
 (segment (start 54.61 44.45) (end 54.61 46.355) (width 0.762) (layer "F.Cu") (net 3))
 (segment (start 100.441353 46.49536) (end 100.7 46.236713) (width 0.254) (layer "F.Cu") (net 3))
 (segment (start 80.01 34.925) (end 82.55 34.925) (width 0.762) (layer "F.Cu") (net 3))
 (segment (start 88.9 46.355) (end 89.95 46.355) (width 0.762) (layer "F.Cu") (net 3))
 (segment (start 69.85 41.91) (end 72.39 44.45) (width 0.762) (layer "F.Cu") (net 3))
 (segment (start 63.5 46.355) (end 63.5 44.45) (width 0.762) (layer "F.Cu") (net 3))
 (segment (start 87.41 40.35) (end 87.41 41.91) (width 0.762) (layer "F.Cu") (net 3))
 (via (at 95.25 37.465) (size 0.6) (drill 0.3) (layers "F.Cu" "B.Cu") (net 3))
 (via (at 100.441353 46.49536) (size 0.6) (drill 0.3) (layers "F.Cu" "B.Cu") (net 3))
 (via (at 101.6 37.465) (size 0.6) (drill 0.3) (layers "F.Cu" "B.Cu") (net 3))
 (segment (start 100.441353 46.49536) (end 100.33 46.384007) (width 0.254) (layer "B.Cu") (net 3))
 (segment (start 103.505 38.735) (end 102.235 37.465) (width 0.762) (layer "B.Cu") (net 3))
 (segment (start 100.33 46.384007) (end 100.33 46.355) (width 0.254) (layer "B.Cu") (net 3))
 (segment (start 102.235 44.45) (end 102.87 43.815) (width 0.762) (layer "B.Cu") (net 3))
 (segment (start 101.6 37.465) (end 95.25 37.465) (width 0.762) (layer "B.Cu") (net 3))
 (segment (start 80.01 39.08) (end 78.74 40.35) (width 0.762) (layer "B.Cu") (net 3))
 (segment (start 102.235 37.465) (end 101.6 37.465) (width 0.762) (layer "B.Cu") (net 3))
 (segment (start 103.505 43.18) (end 103.505 38.735) (width 0.762) (layer "B.Cu") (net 3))
 (segment (start 80.01 34.925) (end 80.01 39.08) (width 0.762) (layer "B.Cu") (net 3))
 (segment (start 100.33 46.355) (end 102.87 43.815) (width 0.254) (layer "B.Cu") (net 3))
 (segment (start 89.95 44.45) (end 102.235 44.45) (width 0.762) (layer "B.Cu") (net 3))
 (segment (start 102.87 43.815) (end 103.505 43.18) (width 0.762) (layer "B.Cu") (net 3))
 (segment (start 59.385 49.53) (end 96.52 49.53) (width 0.254) (layer "F.Cu") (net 15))
 (segment (start 100.05 46) (end 100.05 44.785) (width 0.254) (layer "F.Cu") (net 15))
 (segment (start 57.785 47.93) (end 59.385 49.53) (width 0.254) (layer "F.Cu") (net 15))
 (segment (start 96.52 49.53) (end 100.05 46) (width 0.254) (layer "F.Cu") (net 15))
 (segment (start 95.885 48.895) (end 67.64 48.895) (width 0.254) (layer "F.Cu") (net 11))
 (segment (start 98.75 46.03) (end 95.885 48.895) (width 0.254) (layer "F.Cu") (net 11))
 (segment (start 67.64 48.895) (end 66.675 47.93) (width 0.254) (layer "F.Cu") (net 11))
 (segment (start 98.75 44.785) (end 98.75 46.03) (width 0.254) (layer "F.Cu") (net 11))
 (segment (start 97.1325 46.3325) (end 97.45 46.015) (width 0.254) (layer "F.Cu") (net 10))
 (segment (start 97.45 46.015) (end 97.45 44.785) (width 0.254) (layer "F.Cu") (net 10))
 (via (at 97.1325 46.3325) (size 0.6) (drill 0.3) (layers "F.Cu" "B.Cu") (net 10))
 (via (at 75.565 47.93) (size 0.6) (drill 0.3) (layers "F.Cu" "B.Cu") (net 10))
 (segment (start 76.53 48.895) (end 75.565 47.93) (width 0.254) (layer "B.Cu") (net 10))
 (segment (start 94.57 48.895) (end 76.53 48.895) (width 0.254) (layer "B.Cu") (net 10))
 (segment (start 97.1325 46.3325) (end 94.57 48.895) (width 0.254) (layer "B.Cu") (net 10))
 (segment (start 96.15 44.785) (end 96.15 45.985) (width 0.254) (layer "F.Cu") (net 17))
 (segment (start 96.15 45.985) (end 95.78 46.355) (width 0.254) (layer "F.Cu") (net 17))
 (segment (start 95.78 46.355) (end 95.25 46.355) (width 0.254) (layer "F.Cu") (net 17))
 (via (at 95.25 46.355) (size 0.6) (drill 0.3) (layers "F.Cu" "B.Cu") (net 17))
 (via (at 84.455 47.93) (size 0.6) (drill 0.3) (layers "F.Cu" "B.Cu") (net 17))
 (segment (start 86.03 46.355) (end 95.25 46.355) (width 0.254) (layer "B.Cu") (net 17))
 (segment (start 84.455 47.93) (end 86.03 46.355) (width 0.254) (layer "B.Cu") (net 17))
 (segment (start 100.05 40.285) (end 97.155 43.18) (width 0.254) (layer "F.Cu") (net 4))
 (segment (start 100.05 39.035) (end 100.05 40.285) (width 0.254) (layer "F.Cu") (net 4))
 (segment (start 93.98 46.66) (end 92.71 47.93) (width 0.254) (layer "F.Cu") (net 4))
 (segment (start 97.155 43.18) (end 94.615 43.18) (width 0.254) (layer "F.Cu") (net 4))
 (segment (start 94.615 43.18) (end 93.98 43.815) (width 0.254) (layer "F.Cu") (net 4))
 (segment (start 93.98 43.815) (end 93.98 46.66) (width 0.254) (layer "F.Cu") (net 4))
 (segment (start 96.8 44.785) (end 96.8 45.518054) (width 0.254) (layer "F.Cu") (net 22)))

